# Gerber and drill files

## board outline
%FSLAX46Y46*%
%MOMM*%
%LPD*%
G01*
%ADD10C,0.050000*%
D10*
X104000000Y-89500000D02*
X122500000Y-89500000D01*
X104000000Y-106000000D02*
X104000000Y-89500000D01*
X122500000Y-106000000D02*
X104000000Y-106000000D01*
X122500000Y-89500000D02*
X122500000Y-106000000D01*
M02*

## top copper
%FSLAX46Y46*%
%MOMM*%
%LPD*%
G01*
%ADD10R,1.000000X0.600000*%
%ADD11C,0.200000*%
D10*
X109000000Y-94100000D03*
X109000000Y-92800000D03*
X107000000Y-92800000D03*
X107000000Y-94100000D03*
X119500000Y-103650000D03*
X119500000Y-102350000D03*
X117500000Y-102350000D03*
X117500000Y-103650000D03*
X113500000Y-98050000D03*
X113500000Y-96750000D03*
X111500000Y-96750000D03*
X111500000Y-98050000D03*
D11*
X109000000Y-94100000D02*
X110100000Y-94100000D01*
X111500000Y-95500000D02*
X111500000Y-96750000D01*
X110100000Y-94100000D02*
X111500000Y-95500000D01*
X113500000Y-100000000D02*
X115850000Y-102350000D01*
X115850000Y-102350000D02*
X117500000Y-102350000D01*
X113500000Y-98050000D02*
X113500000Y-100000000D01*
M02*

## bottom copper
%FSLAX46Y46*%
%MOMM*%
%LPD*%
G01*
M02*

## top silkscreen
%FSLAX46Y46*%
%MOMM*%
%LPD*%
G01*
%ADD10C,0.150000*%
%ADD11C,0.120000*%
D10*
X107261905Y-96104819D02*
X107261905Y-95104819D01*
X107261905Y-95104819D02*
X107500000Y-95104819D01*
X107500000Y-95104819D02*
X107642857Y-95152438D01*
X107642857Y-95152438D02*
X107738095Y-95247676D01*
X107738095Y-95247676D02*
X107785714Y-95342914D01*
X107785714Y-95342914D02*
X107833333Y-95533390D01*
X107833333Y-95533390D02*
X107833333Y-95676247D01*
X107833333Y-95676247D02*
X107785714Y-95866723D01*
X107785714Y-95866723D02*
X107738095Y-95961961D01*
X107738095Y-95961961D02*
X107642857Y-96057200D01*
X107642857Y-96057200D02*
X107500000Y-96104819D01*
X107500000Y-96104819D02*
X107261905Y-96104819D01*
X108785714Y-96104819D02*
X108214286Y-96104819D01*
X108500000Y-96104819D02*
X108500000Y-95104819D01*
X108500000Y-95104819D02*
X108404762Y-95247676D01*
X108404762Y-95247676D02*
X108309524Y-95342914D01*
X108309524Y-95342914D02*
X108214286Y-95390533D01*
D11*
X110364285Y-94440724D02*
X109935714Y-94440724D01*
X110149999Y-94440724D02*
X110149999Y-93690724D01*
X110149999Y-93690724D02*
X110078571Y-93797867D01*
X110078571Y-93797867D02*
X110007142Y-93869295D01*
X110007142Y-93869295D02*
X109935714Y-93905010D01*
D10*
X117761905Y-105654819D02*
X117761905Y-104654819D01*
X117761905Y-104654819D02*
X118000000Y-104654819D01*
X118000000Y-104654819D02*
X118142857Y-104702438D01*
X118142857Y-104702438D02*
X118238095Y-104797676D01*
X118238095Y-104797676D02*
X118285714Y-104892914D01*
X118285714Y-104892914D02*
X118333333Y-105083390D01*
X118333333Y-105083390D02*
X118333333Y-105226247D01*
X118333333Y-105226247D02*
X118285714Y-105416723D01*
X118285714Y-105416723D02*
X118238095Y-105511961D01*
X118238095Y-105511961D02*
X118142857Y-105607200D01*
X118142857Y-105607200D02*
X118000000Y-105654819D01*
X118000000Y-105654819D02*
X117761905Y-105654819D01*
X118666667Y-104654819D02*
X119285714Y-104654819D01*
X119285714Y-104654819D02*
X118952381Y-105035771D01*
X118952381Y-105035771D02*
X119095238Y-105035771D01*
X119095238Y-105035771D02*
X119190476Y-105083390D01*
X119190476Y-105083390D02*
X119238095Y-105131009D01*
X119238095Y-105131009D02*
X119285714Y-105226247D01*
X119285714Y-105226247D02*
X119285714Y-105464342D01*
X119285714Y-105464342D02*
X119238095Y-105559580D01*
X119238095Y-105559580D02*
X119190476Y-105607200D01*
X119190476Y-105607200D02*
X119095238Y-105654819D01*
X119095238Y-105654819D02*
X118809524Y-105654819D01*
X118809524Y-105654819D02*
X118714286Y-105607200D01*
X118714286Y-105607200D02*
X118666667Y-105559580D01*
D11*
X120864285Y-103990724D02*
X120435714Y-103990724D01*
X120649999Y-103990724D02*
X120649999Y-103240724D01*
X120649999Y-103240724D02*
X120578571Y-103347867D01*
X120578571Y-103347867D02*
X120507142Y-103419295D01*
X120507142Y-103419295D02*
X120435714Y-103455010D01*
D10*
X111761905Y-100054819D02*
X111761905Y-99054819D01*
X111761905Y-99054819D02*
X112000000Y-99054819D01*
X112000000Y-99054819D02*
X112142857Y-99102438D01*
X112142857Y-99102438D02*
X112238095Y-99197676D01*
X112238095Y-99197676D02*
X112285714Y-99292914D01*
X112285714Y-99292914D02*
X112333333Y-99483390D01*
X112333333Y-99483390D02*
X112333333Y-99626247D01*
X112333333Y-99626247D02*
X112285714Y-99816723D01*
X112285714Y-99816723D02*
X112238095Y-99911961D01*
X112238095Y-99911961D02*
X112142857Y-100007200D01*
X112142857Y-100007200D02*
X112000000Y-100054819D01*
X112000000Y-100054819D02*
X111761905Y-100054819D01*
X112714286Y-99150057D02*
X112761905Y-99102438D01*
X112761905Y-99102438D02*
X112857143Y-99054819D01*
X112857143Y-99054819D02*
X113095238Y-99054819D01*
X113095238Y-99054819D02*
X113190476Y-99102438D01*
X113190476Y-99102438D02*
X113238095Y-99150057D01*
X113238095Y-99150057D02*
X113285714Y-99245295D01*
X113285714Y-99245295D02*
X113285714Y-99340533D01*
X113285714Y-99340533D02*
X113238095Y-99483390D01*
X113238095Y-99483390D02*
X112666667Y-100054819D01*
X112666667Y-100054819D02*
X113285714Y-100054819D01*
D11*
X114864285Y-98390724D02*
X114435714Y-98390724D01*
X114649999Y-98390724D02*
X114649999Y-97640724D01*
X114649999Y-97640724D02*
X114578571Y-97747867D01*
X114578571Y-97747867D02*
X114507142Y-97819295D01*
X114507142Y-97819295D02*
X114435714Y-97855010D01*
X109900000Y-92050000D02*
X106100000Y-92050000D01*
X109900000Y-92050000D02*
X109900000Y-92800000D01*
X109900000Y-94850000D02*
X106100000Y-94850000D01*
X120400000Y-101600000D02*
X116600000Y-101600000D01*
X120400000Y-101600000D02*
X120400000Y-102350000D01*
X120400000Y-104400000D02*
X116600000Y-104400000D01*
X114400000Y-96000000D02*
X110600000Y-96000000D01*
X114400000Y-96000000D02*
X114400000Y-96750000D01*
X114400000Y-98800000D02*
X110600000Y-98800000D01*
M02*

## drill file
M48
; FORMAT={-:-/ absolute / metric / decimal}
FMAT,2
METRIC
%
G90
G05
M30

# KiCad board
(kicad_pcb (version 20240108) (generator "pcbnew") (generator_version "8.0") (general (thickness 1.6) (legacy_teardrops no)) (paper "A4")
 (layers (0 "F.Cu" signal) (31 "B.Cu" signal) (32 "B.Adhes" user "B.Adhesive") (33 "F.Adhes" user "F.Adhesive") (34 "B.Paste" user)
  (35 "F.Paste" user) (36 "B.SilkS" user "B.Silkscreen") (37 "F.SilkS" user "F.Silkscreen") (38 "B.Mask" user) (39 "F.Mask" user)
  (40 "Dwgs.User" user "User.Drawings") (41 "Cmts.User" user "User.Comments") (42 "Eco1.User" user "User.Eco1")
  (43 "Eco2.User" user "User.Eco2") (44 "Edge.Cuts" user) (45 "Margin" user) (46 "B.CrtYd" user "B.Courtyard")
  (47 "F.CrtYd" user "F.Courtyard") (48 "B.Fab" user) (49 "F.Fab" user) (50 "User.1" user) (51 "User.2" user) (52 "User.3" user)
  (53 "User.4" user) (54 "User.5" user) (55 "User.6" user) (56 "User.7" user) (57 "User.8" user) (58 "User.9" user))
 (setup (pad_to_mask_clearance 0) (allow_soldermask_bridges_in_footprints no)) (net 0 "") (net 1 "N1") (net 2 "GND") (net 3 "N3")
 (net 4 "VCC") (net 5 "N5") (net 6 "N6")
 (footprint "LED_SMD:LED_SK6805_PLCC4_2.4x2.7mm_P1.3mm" (layer "F.Cu") (at 108 93.45 180)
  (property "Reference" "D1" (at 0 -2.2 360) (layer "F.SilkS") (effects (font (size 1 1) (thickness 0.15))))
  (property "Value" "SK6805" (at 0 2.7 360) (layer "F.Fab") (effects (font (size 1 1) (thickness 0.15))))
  (fp_line (start -1.9 1.4) (end 1.9 1.4) (stroke (width 0.12) (type solid)) (layer "F.SilkS"))
  (fp_line (start -1.9 1.4) (end -1.9 0.65) (stroke (width 0.12) (type solid)) (layer "F.SilkS"))
  (fp_line (start -1.9 -1.4) (end 1.9 -1.4) (stroke (width 0.12) (type solid)) (layer "F.SilkS"))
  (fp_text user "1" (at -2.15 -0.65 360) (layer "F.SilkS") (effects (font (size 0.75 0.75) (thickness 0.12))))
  (pad "1" smd rect (at -1 -0.65 180) (size 1 0.6) (layers "F.Cu" "F.Paste" "F.Mask") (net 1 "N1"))
  (pad "2" smd rect (at -1 0.65 180) (size 1 0.6) (layers "F.Cu" "F.Paste" "F.Mask") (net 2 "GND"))
  (pad "3" smd rect (at 1 0.65 180) (size 1 0.6) (layers "F.Cu" "F.Paste" "F.Mask") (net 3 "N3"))
  (pad "4" smd rect (at 1 -0.65 180) (size 1 0.6) (layers "F.Cu" "F.Paste" "F.Mask") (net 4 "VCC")))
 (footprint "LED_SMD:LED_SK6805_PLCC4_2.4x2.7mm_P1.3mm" (layer "F.Cu") (at 118.5 103 180)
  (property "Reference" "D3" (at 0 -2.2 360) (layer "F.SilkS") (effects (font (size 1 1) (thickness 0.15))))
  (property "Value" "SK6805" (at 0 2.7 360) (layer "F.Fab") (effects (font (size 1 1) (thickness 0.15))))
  (fp_line (start -1.9 1.4) (end 1.9 1.4) (stroke (width 0.12) (type solid)) (layer "F.SilkS"))
  (fp_line (start -1.9 1.4) (end -1.9 0.65) (stroke (width 0.12) (type solid)) (layer "F.SilkS"))
  (fp_line (start -1.9 -1.4) (end 1.9 -1.4) (stroke (width 0.12) (type solid)) (layer "F.SilkS"))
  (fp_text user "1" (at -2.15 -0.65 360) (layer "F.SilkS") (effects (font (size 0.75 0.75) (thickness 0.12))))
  (pad "1" smd rect (at -1 -0.65 180) (size 1 0.6) (layers "F.Cu" "F.Paste" "F.Mask") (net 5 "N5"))
  (pad "2" smd rect (at -1 0.65 180) (size 1 0.6) (layers "F.Cu" "F.Paste" "F.Mask") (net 2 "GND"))
  (pad "3" smd rect (at 1 0.65 180) (size 1 0.6) (layers "F.Cu" "F.Paste" "F.Mask") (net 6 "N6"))
  (pad "4" smd rect (at 1 -0.65 180) (size 1 0.6) (layers "F.Cu" "F.Paste" "F.Mask") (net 4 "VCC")))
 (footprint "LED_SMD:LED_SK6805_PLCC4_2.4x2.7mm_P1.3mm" (layer "F.Cu") (at 112.5 97.4 180)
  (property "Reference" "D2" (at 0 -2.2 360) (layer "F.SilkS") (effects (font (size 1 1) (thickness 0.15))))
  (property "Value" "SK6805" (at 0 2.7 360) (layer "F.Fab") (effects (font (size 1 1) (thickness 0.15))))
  (fp_line (start -1.9 1.4) (end 1.9 1.4) (stroke (width 0.12) (type solid)) (layer "F.SilkS"))
  (fp_line (start -1.9 1.4) (end -1.9 0.65) (stroke (width 0.12) (type solid)) (layer "F.SilkS"))
  (fp_line (start -1.9 -1.4) (end 1.9 -1.4) (stroke (width 0.12) (type solid)) (layer "F.SilkS"))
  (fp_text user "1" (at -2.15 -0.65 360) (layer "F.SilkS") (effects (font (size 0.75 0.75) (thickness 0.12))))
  (pad "1" smd rect (at -1 -0.65 180) (size 1 0.6) (layers "F.Cu" "F.Paste" "F.Mask") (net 6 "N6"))
  (pad "2" smd rect (at -1 0.65 180) (size 1 0.6) (layers "F.Cu" "F.Paste" "F.Mask") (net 2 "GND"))
  (pad "3" smd rect (at 1 0.65 180) (size 1 0.6) (layers "F.Cu" "F.Paste" "F.Mask") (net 1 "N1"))
  (pad "4" smd rect (at 1 -0.65 180) (size 1 0.6) (layers "F.Cu" "F.Paste" "F.Mask") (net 4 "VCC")))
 (gr_line (start 104 89.5) (end 122.5 89.5) (stroke (width 0.05) (type default)) (layer "Edge.Cuts"))
 (gr_line (start 104 106) (end 104 89.5) (stroke (width 0.05) (type default)) (layer "Edge.Cuts"))
 (gr_line (start 122.5 106) (end 104 106) (stroke (width 0.05) (type default)) (layer "Edge.Cuts"))
 (gr_line (start 122.5 89.5) (end 122.5 106) (stroke (width 0.05) (type default)) (layer "Edge.Cuts"))
 (segment (start 109 94.1) (end 110.1 94.1) (width 0.2) (layer "F.Cu") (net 1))
 (segment (start 111.5 95.5) (end 111.5 96.75) (width 0.2) (layer "F.Cu") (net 1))
 (segment (start 110.1 94.1) (end 111.5 95.5) (width 0.2) (layer "F.Cu") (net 1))
 (segment (start 113.5 100) (end 115.85 102.35) (width 0.2) (layer "F.Cu") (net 6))
 (segment (start 115.85 102.35) (end 117.5 102.35) (width 0.2) (layer "F.Cu") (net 6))
 (segment (start 113.5 98.05) (end 113.5 100) (width 0.2) (layer "F.Cu") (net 6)))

